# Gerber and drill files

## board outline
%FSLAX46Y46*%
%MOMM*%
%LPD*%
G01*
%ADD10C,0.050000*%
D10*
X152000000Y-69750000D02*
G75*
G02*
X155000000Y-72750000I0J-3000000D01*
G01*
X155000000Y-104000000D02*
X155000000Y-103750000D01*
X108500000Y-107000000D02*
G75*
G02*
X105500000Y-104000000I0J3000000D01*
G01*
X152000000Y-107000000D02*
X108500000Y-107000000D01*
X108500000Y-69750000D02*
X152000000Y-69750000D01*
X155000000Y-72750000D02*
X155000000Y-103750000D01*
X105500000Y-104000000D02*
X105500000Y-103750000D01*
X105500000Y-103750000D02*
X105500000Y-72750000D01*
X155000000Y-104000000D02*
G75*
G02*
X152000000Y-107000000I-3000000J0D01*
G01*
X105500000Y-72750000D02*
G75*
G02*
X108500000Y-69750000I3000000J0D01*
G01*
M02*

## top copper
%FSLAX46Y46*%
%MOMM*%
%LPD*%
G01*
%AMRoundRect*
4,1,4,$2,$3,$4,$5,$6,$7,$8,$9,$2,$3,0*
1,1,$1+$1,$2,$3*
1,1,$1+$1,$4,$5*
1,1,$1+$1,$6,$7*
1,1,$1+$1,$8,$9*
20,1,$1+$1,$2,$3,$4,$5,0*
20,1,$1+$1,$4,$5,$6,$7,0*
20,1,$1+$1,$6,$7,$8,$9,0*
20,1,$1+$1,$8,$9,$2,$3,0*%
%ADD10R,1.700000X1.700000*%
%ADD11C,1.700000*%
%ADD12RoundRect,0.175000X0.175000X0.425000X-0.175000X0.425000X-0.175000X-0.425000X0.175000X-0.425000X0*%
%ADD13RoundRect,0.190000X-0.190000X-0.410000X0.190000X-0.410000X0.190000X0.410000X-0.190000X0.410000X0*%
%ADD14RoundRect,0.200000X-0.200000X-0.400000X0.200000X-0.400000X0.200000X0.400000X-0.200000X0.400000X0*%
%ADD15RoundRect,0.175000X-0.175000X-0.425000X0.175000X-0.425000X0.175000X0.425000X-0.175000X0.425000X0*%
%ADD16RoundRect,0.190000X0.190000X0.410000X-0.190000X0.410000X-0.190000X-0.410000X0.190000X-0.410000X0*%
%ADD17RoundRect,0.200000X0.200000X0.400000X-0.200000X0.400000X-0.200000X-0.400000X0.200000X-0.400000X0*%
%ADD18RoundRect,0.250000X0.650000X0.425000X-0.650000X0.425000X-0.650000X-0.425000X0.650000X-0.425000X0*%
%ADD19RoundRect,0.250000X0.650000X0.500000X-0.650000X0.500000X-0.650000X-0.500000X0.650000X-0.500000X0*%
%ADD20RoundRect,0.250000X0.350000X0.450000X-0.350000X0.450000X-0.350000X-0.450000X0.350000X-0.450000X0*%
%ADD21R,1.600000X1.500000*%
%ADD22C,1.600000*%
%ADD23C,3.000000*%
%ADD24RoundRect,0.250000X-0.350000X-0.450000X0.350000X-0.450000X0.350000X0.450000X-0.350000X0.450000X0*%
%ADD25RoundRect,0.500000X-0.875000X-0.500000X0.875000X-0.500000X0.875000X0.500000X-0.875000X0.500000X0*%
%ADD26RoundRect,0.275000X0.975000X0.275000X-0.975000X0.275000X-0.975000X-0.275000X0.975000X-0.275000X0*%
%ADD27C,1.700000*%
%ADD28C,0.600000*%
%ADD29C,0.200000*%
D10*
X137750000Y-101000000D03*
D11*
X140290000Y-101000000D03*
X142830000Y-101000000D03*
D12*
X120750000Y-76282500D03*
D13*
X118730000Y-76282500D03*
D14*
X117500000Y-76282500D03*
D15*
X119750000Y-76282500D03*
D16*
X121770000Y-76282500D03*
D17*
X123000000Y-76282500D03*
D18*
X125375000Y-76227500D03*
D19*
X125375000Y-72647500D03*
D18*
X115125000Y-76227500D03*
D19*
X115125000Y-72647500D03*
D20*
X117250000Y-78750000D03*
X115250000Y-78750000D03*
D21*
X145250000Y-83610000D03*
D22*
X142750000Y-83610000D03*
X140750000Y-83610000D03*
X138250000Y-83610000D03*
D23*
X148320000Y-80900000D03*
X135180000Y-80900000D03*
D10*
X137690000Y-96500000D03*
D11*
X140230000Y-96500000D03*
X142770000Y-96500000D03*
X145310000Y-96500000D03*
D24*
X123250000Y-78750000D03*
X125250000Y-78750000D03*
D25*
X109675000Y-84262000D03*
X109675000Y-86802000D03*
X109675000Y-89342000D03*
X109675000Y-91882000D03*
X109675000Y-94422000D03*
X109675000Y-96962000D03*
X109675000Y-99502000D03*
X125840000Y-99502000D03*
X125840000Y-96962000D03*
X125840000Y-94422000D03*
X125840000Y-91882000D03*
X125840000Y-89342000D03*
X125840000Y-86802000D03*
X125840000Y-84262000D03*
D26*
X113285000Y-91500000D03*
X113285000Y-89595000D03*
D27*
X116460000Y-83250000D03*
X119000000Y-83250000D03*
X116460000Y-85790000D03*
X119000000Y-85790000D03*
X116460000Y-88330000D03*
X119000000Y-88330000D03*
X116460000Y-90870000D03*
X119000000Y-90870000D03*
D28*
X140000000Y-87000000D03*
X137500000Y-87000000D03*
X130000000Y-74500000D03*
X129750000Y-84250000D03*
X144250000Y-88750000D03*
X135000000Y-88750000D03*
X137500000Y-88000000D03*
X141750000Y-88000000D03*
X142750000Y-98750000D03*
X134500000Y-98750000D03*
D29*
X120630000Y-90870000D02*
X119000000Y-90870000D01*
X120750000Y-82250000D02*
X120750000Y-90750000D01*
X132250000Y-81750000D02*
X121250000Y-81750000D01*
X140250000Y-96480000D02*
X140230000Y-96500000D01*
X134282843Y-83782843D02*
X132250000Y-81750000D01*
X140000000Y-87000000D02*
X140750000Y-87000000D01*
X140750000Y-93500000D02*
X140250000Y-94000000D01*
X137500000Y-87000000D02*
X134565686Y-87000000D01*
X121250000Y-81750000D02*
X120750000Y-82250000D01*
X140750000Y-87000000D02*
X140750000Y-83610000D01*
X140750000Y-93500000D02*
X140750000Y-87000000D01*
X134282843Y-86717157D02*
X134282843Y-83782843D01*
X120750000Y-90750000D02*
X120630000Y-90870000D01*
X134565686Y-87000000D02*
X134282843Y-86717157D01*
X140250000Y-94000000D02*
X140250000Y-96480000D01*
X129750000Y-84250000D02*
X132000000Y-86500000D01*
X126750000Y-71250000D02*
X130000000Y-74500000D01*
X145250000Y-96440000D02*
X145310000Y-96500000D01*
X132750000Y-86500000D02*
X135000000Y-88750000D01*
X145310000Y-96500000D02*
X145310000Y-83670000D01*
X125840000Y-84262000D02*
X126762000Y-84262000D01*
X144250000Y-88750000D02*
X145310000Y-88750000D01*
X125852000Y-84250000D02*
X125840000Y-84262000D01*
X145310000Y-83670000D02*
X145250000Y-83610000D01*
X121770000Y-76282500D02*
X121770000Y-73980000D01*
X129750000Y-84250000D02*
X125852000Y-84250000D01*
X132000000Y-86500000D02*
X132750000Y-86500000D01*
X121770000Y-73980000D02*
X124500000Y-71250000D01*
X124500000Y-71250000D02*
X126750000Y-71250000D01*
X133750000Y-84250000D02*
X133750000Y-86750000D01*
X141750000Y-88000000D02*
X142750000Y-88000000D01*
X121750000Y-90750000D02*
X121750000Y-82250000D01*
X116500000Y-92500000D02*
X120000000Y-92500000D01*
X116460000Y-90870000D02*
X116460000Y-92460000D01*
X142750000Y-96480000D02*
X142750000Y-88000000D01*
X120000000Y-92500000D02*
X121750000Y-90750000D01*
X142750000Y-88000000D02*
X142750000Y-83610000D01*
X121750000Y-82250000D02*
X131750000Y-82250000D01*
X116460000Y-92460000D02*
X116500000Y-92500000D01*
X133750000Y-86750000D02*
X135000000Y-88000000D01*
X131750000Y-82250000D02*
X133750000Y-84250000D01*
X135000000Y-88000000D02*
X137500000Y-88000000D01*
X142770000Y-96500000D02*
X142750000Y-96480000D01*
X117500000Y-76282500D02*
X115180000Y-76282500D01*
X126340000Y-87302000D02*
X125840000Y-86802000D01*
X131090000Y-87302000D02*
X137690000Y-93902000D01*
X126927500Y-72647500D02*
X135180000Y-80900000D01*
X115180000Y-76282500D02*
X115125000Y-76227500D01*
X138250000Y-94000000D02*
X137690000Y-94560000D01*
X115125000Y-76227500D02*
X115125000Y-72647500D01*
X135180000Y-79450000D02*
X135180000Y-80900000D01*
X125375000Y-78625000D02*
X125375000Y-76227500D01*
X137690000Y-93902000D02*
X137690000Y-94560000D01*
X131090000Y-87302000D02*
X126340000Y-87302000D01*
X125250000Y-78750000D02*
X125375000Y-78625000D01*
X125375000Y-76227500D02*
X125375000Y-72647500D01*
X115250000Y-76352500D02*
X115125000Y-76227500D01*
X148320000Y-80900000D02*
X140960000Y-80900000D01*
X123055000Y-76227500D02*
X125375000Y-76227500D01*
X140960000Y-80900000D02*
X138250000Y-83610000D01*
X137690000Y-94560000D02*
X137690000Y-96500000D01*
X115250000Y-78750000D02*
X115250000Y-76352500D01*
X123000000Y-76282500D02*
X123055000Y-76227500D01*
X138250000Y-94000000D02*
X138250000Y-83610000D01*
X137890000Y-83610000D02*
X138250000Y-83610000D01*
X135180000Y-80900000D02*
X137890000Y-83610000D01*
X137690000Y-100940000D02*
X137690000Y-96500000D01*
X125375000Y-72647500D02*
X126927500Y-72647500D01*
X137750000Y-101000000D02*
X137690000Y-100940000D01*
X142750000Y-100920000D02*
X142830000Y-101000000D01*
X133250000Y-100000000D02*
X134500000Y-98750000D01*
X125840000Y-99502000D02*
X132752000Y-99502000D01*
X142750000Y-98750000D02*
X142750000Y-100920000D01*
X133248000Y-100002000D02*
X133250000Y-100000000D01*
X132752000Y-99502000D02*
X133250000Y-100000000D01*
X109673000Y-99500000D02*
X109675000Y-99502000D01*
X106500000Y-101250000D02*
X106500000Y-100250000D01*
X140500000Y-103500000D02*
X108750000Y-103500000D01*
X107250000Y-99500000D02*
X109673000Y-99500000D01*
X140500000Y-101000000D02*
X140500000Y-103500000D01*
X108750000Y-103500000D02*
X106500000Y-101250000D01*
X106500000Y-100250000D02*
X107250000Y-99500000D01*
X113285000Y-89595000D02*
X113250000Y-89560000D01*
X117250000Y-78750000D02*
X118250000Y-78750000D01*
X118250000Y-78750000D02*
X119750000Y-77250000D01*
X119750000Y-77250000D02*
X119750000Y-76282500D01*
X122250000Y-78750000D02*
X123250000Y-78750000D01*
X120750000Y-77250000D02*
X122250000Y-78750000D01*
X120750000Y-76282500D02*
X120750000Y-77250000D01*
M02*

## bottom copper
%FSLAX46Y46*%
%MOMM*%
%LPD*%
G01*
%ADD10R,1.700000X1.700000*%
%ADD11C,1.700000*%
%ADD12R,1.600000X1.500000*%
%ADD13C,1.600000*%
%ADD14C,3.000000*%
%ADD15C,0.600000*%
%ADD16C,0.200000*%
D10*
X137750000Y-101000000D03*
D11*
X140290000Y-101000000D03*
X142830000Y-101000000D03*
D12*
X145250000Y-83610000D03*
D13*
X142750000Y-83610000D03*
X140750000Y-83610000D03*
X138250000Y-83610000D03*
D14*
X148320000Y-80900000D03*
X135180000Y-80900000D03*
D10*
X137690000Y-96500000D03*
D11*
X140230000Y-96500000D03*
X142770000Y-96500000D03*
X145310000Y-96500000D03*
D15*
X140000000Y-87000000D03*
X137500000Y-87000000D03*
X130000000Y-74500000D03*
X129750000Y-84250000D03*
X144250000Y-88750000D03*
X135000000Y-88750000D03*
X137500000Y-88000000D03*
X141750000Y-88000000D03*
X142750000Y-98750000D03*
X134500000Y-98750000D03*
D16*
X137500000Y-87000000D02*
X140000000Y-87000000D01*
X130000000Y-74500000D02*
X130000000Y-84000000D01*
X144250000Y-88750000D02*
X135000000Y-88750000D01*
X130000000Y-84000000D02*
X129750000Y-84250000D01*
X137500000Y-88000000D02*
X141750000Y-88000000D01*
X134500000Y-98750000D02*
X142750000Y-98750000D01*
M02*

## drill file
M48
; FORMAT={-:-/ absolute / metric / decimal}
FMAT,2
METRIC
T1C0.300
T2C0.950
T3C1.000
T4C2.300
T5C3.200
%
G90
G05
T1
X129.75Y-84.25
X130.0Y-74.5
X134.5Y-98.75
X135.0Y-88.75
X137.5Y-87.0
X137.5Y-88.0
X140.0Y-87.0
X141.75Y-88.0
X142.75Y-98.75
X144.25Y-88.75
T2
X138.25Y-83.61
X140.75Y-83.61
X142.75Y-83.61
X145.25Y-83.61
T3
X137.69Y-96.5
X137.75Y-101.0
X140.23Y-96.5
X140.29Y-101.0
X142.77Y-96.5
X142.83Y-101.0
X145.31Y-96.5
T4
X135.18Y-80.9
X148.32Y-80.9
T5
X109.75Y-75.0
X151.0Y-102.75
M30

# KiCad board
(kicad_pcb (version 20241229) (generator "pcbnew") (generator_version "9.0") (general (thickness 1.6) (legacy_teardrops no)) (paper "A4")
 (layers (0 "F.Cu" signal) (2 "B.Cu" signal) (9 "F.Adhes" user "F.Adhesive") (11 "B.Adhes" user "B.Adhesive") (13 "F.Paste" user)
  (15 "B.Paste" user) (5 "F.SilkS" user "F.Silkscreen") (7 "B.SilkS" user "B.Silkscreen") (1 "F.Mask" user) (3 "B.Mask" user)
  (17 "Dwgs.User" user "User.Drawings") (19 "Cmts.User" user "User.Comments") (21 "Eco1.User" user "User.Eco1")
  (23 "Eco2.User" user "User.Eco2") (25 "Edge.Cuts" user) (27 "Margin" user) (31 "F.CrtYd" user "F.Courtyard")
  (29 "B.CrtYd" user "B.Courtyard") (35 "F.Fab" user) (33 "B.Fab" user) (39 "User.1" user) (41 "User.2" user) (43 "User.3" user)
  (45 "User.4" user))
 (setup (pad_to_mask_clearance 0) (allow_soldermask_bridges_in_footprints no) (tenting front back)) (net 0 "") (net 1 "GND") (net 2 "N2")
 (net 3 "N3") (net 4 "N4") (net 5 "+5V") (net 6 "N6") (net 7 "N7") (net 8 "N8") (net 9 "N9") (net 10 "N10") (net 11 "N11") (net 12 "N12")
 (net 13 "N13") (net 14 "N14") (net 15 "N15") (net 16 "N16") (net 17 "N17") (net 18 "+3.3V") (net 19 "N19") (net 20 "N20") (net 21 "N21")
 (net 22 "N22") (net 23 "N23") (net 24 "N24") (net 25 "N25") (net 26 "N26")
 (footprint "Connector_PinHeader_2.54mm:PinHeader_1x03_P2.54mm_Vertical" (layer "F.Cu") (at 137.75 101 90)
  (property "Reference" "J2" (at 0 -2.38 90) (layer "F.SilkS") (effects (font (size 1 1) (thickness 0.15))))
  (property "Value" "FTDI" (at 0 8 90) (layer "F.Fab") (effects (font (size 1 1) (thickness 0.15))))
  (pad "1" thru_hole rect (at 0 0 90) (size 1.7 1.7) (drill 1) (layers "*.Cu" "*.Mask") (remove_unused_layers no) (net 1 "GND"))
  (pad "2" thru_hole circle (at 0 2.54 90) (size 1.7 1.7) (drill 1) (layers "*.Cu" "*.Mask") (remove_unused_layers no) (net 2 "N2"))
  (pad "3" thru_hole circle (at 0 5.08 90) (size 1.7 1.7) (drill 1) (layers "*.Cu" "*.Mask") (remove_unused_layers no) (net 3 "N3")))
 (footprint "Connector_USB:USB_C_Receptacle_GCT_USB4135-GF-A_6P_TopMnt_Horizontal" (layer "F.Cu") (at 120.25 73.25 180)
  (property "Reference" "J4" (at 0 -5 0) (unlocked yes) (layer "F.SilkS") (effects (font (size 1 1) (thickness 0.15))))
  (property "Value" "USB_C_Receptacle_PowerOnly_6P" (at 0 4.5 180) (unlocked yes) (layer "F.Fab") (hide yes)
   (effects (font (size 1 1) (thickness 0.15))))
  (pad "A5" smd roundrect (at -0.5 -3.0325 180) (size 0.7 1.2) (layers "F.Cu" "F.Mask" "F.Paste") (roundrect_rratio 0.25) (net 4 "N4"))
  (pad "A9" smd roundrect (at 1.52 -3.0325) (size 0.76 1.2) (layers "F.Cu" "F.Mask" "F.Paste") (roundrect_rratio 0.25) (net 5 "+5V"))
  (pad "A12" smd roundrect (at 2.75 -3.0325) (size 0.8 1.2) (layers "F.Cu" "F.Mask" "F.Paste") (roundrect_rratio 0.25) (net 1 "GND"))
  (pad "B5" smd roundrect (at 0.5 -3.0325) (size 0.7 1.2) (layers "F.Cu" "F.Mask" "F.Paste") (roundrect_rratio 0.25) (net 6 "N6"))
  (pad "B9" smd roundrect (at -1.52 -3.0325 180) (size 0.76 1.2) (layers "F.Cu" "F.Mask" "F.Paste") (roundrect_rratio 0.25) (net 5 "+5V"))
  (pad "B12" smd roundrect (at -2.75 -3.0325 180) (size 0.8 1.2) (layers "F.Cu" "F.Mask" "F.Paste") (roundrect_rratio 0.25) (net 1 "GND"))
  (pad "S1" smd roundrect (at -5.125 -2.9775 180) (size 1.8 1.35) (layers "F.Cu" "F.Mask" "F.Paste") (roundrect_rratio 0.1851851852)
   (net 1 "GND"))
  (pad "S1" smd roundrect (at -5.125 0.6025 180) (size 1.8 1.5) (layers "F.Cu" "F.Mask" "F.Paste") (roundrect_rratio 0.1666666667)
   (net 1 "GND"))
  (pad "S1" smd roundrect (at 5.125 -2.9775 180) (size 1.8 1.35) (layers "F.Cu" "F.Mask" "F.Paste") (roundrect_rratio 0.1851851852)
   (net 1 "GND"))
  (pad "S1" smd roundrect (at 5.125 0.6025 180) (size 1.8 1.5) (layers "F.Cu" "F.Mask" "F.Paste") (roundrect_rratio 0.1666666667)
   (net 1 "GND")))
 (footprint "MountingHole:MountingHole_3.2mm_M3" (layer "F.Cu") (at 151 102.75)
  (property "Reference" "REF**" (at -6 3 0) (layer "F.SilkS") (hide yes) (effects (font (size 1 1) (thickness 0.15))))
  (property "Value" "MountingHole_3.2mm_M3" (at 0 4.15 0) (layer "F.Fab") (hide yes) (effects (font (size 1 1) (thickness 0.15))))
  (pad "" np_thru_hole circle (at 0 0) (size 3.2 3.2) (drill 3.2) (layers "*.Cu" "*.Mask")))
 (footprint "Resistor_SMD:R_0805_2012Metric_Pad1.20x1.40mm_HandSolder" (layer "F.Cu") (at 116.25 78.75 180)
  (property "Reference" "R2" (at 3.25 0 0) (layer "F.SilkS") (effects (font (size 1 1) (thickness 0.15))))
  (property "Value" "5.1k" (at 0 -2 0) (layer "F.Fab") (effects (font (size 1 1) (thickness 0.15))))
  (pad "1" smd roundrect (at -1 0 180) (size 1.2 1.4) (layers "F.Cu" "F.Mask" "F.Paste") (roundrect_rratio 0.208333) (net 6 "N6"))
  (pad "2" smd roundrect (at 1 0 180) (size 1.2 1.4) (layers "F.Cu" "F.Mask" "F.Paste") (roundrect_rratio 0.208333) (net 1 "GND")))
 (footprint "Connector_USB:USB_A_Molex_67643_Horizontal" (layer "F.Cu") (at 145.25 83.61 180)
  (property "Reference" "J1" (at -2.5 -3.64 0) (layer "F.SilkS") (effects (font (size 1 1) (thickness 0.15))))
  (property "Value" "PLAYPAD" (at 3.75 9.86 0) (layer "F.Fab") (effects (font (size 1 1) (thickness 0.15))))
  (pad "1" thru_hole rect (at 0 0 180) (size 1.6 1.5) (drill 0.95) (layers "*.Cu" "*.Mask") (remove_unused_layers no) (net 5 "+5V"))
  (pad "2" thru_hole circle (at 2.5 0 180) (size 1.6 1.6) (drill 0.95) (layers "*.Cu" "*.Mask") (remove_unused_layers no) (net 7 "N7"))
  (pad "3" thru_hole circle (at 4.5 0 180) (size 1.6 1.6) (drill 0.95) (layers "*.Cu" "*.Mask") (remove_unused_layers no) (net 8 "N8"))
  (pad "4" thru_hole circle (at 7 0 180) (size 1.6 1.6) (drill 0.95) (layers "*.Cu" "*.Mask") (remove_unused_layers no) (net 1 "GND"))
  (pad "5" thru_hole circle (at -3.07 2.71 180) (size 3 3) (drill 2.3) (layers "*.Cu" "*.Mask") (remove_unused_layers no) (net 1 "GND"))
  (pad "5" thru_hole circle (at 10.07 2.71 180) (size 3 3) (drill 2.3) (layers "*.Cu" "*.Mask") (remove_unused_layers no) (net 1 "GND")))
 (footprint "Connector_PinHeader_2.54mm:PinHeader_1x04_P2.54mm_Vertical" (layer "F.Cu") (at 137.69 96.5 90)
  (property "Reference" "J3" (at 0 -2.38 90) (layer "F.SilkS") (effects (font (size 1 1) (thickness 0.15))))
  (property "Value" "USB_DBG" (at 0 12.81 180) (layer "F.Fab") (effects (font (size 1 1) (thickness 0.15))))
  (pad "1" thru_hole rect (at 0 0 90) (size 1.7 1.7) (drill 1) (layers "*.Cu" "*.Mask") (remove_unused_layers no) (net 1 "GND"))
  (pad "2" thru_hole circle (at 0 2.54 90) (size 1.7 1.7) (drill 1) (layers "*.Cu" "*.Mask") (remove_unused_layers no) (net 8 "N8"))
  (pad "3" thru_hole circle (at 0 5.08 90) (size 1.7 1.7) (drill 1) (layers "*.Cu" "*.Mask") (remove_unused_layers no) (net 7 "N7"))
  (pad "4" thru_hole circle (at 0 7.62 90) (size 1.7 1.7) (drill 1) (layers "*.Cu" "*.Mask") (remove_unused_layers no) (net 5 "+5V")))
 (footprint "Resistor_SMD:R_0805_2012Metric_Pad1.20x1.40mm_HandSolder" (layer "F.Cu") (at 124.25 78.75)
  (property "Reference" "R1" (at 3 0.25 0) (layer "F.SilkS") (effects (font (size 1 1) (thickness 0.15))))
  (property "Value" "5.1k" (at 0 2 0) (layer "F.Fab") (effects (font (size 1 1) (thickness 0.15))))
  (pad "1" smd roundrect (at -1 0) (size 1.2 1.4) (layers "F.Cu" "F.Mask" "F.Paste") (roundrect_rratio 0.208333) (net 4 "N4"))
  (pad "2" smd roundrect (at 1 0) (size 1.2 1.4) (layers "F.Cu" "F.Mask" "F.Paste") (roundrect_rratio 0.208333) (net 1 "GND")))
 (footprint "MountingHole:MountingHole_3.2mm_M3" (layer "F.Cu") (at 109.75 75)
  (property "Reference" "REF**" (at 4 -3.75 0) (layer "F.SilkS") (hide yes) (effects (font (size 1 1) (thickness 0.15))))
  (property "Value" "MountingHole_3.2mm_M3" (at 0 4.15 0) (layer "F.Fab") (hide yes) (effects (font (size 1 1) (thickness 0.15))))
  (pad "" np_thru_hole circle (at 0 0) (size 3.2 3.2) (drill 3.2) (layers "*.Cu" "*.Mask")))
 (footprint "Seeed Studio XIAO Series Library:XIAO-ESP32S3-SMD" (layer "F.Cu") (at 117.736364 91.835)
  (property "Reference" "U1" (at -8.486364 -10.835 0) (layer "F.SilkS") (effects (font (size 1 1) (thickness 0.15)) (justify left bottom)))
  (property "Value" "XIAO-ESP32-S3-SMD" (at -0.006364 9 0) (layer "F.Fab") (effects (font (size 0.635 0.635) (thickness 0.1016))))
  (pad "1" smd roundrect (at -8.061364 -7.573) (size 2.75 2) (layers "F.Cu" "F.Mask" "F.Paste") (roundrect_rratio 0.25) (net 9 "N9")
   (solder_mask_margin 0.0508) (thermal_bridge_angle 45))
  (pad "2" smd roundrect (at -8.061364 -5.033) (size 2.75 2) (layers "F.Cu" "F.Mask" "F.Paste") (roundrect_rratio 0.25) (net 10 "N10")
   (solder_mask_margin 0.0508) (thermal_bridge_angle 45))
  (pad "3" smd roundrect (at -8.061364 -2.493) (size 2.75 2) (layers "F.Cu" "F.Mask" "F.Paste") (roundrect_rratio 0.25) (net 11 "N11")
   (solder_mask_margin 0.0508) (thermal_bridge_angle 45))
  (pad "4" smd roundrect (at -8.061364 0.047) (size 2.75 2) (layers "F.Cu" "F.Mask" "F.Paste") (roundrect_rratio 0.25) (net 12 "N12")
   (solder_mask_margin 0.0508) (thermal_bridge_angle 45))
  (pad "5" smd roundrect (at -8.061364 2.587) (size 2.75 2) (layers "F.Cu" "F.Mask" "F.Paste") (roundrect_rratio 0.25) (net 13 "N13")
   (solder_mask_margin 0.0508) (thermal_bridge_angle 45))
  (pad "6" smd roundrect (at -8.061364 5.127) (size 2.75 2) (layers "F.Cu" "F.Mask" "F.Paste") (roundrect_rratio 0.25) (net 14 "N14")
   (solder_mask_margin 0.0508) (thermal_bridge_angle 45))
  (pad "7" smd roundrect (at -8.061364 7.667) (size 2.75 2) (layers "F.Cu" "F.Mask" "F.Paste") (roundrect_rratio 0.25) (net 2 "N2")
   (solder_mask_margin 0.0508) (thermal_bridge_angle 45))
  (pad "8" smd roundrect (at 8.103636 7.667) (size 2.75 2) (layers "F.Cu" "F.Mask" "F.Paste") (roundrect_rratio 0.25) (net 3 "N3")
   (solder_mask_margin 0.0508) (thermal_bridge_angle 45))
  (pad "9" smd roundrect (at 8.103636 5.127) (size 2.75 2) (layers "F.Cu" "F.Mask" "F.Paste") (roundrect_rratio 0.25) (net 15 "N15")
   (solder_mask_margin 0.0508) (thermal_bridge_angle 45))
  (pad "10" smd roundrect (at 8.103636 2.587) (size 2.75 2) (layers "F.Cu" "F.Mask" "F.Paste") (roundrect_rratio 0.25) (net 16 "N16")
   (solder_mask_margin 0.0508) (thermal_bridge_angle 45))
  (pad "11" smd roundrect (at 8.103636 0.047) (size 2.75 2) (layers "F.Cu" "F.Mask" "F.Paste") (roundrect_rratio 0.25) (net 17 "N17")
   (solder_mask_margin 0.0508) (thermal_bridge_angle 45))
  (pad "12" smd roundrect (at 8.103636 -2.493) (size 2.75 2) (layers "F.Cu" "F.Mask" "F.Paste") (roundrect_rratio 0.25) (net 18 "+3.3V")
   (solder_mask_margin 0.0508) (thermal_bridge_angle 45))
  (pad "13" smd roundrect (at 8.103636 -5.033) (size 2.75 2) (layers "F.Cu" "F.Mask" "F.Paste") (roundrect_rratio 0.25) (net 1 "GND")
   (solder_mask_margin 0.0508) (thermal_bridge_angle 45))
  (pad "14" smd roundrect (at 8.103636 -7.573) (size 2.75 2) (layers "F.Cu" "F.Mask" "F.Paste") (roundrect_rratio 0.25) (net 5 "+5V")
   (solder_mask_margin 0.0508) (thermal_bridge_angle 45))
  (pad "15" smd roundrect (at -4.451364 -0.335 180) (size 2.5 1.1) (layers "F.Cu" "F.Mask" "F.Paste") (roundrect_rratio 0.25) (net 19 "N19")
   (solder_mask_margin 0.0508) (thermal_bridge_angle 45))
  (pad "16" smd roundrect (at -4.451364 -2.24 180) (size 2.5 1.1) (layers "F.Cu" "F.Mask" "F.Paste") (roundrect_rratio 0.25) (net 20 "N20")
   (solder_mask_margin 0.0508) (thermal_bridge_angle 45))
  (pad "17" smd circle (at -1.276364 -8.585) (size 1.7 1.7) (layers "F.Cu" "F.Mask" "F.Paste") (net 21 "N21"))
  (pad "18" smd circle (at 1.263636 -8.585) (size 1.7 1.7) (layers "F.Cu" "F.Mask" "F.Paste") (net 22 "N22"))
  (pad "19" smd circle (at -1.276364 -6.045) (size 1.7 1.7) (layers "F.Cu" "F.Mask" "F.Paste") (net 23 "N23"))
  (pad "20" smd circle (at 1.263636 -6.045) (size 1.7 1.7) (layers "F.Cu" "F.Mask" "F.Paste") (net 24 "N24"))
  (pad "21" smd circle (at -1.276364 -3.505) (size 1.7 1.7) (layers "F.Cu" "F.Mask" "F.Paste") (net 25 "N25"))
  (pad "22" smd circle (at 1.263636 -3.505) (size 1.7 1.7) (layers "F.Cu" "F.Mask" "F.Paste") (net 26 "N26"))
  (pad "23" smd circle (at -1.276364 -0.965) (size 1.7 1.7) (layers "F.Cu" "F.Mask" "F.Paste") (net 7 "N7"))
  (pad "24" smd circle (at 1.263636 -0.965) (size 1.7 1.7) (layers "F.Cu" "F.Mask" "F.Paste") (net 8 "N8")))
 (gr_arc (start 152 69.75) (mid 154.12132 70.62868) (end 155 72.75) (stroke (width 0.05) (type default)) (layer "Edge.Cuts"))
 (gr_line (start 155 104) (end 155 103.75) (stroke (width 0.05) (type default)) (layer "Edge.Cuts"))
 (gr_arc (start 108.5 107) (mid 106.37868 106.12132) (end 105.5 104) (stroke (width 0.05) (type default)) (layer "Edge.Cuts"))
 (gr_line (start 152 107) (end 108.5 107) (stroke (width 0.05) (type default)) (layer "Edge.Cuts"))
 (gr_line (start 108.5 69.75) (end 152 69.75) (stroke (width 0.05) (type default)) (layer "Edge.Cuts"))
 (gr_line (start 155 72.75) (end 155 103.75) (stroke (width 0.05) (type default)) (layer "Edge.Cuts"))
 (gr_line (start 105.5 104) (end 105.5 103.75) (stroke (width 0.05) (type default)) (layer "Edge.Cuts"))
 (gr_line (start 105.5 103.75) (end 105.5 72.75) (stroke (width 0.05) (type default)) (layer "Edge.Cuts"))
 (gr_arc (start 155 104) (mid 154.12132 106.12132) (end 152 107) (stroke (width 0.05) (type default)) (layer "Edge.Cuts"))
 (gr_arc (start 105.5 72.75) (mid 106.37868 70.62868) (end 108.5 69.75) (stroke (width 0.05) (type default)) (layer "Edge.Cuts"))
 (segment (start 120.63 90.87) (end 119 90.87) (width 0.2) (layer "F.Cu") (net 8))
 (segment (start 120.75 82.25) (end 120.75 90.75) (width 0.2) (layer "F.Cu") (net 8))
 (segment (start 132.25 81.75) (end 121.25 81.75) (width 0.2) (layer "F.Cu") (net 8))
 (segment (start 140.25 96.48) (end 140.23 96.5) (width 0.2) (layer "F.Cu") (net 8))
 (segment (start 134.282843 83.782843) (end 132.25 81.75) (width 0.2) (layer "F.Cu") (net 8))
 (segment (start 140 87) (end 140.75 87) (width 0.2) (layer "F.Cu") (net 8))
 (segment (start 140.75 93.5) (end 140.25 94) (width 0.2) (layer "F.Cu") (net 8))
 (segment (start 137.5 87) (end 134.565686 87) (width 0.2) (layer "F.Cu") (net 8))
 (segment (start 121.25 81.75) (end 120.75 82.25) (width 0.2) (layer "F.Cu") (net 8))
 (segment (start 140.75 87) (end 140.75 83.61) (width 0.2) (layer "F.Cu") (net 8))
 (segment (start 140.75 93.5) (end 140.75 87) (width 0.2) (layer "F.Cu") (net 8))
 (segment (start 134.282843 86.717157) (end 134.282843 83.782843) (width 0.2) (layer "F.Cu") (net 8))
 (segment (start 120.75 90.75) (end 120.63 90.87) (width 0.2) (layer "F.Cu") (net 8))
 (segment (start 134.565686 87) (end 134.282843 86.717157) (width 0.2) (layer "F.Cu") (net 8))
 (segment (start 140.25 94) (end 140.25 96.48) (width 0.2) (layer "F.Cu") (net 8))
 (via (at 140 87) (size 0.6) (drill 0.3) (layers "F.Cu" "B.Cu") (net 8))
 (via (at 137.5 87) (size 0.6) (drill 0.3) (layers "F.Cu" "B.Cu") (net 8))
 (segment (start 137.5 87) (end 140 87) (width 0.2) (layer "B.Cu") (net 8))
 (segment (start 129.75 84.25) (end 132 86.5) (width 0.2) (layer "F.Cu") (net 5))
 (segment (start 126.75 71.25) (end 130 74.5) (width 0.2) (layer "F.Cu") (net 5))
 (segment (start 145.25 96.44) (end 145.31 96.5) (width 0.2) (layer "F.Cu") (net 5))
 (segment (start 132.75 86.5) (end 135 88.75) (width 0.2) (layer "F.Cu") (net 5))
 (segment (start 145.31 96.5) (end 145.31 83.67) (width 0.2) (layer "F.Cu") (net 5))
 (segment (start 125.84 84.262) (end 126.762 84.262) (width 0.2) (layer "F.Cu") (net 5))
 (segment (start 144.25 88.75) (end 145.31 88.75) (width 0.2) (layer "F.Cu") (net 5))
 (segment (start 125.852 84.25) (end 125.84 84.262) (width 0.2) (layer "F.Cu") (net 5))
 (segment (start 145.31 83.67) (end 145.25 83.61) (width 0.2) (layer "F.Cu") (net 5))
 (segment (start 121.77 76.2825) (end 121.77 73.98) (width 0.2) (layer "F.Cu") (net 5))
 (segment (start 129.75 84.25) (end 125.852 84.25) (width 0.2) (layer "F.Cu") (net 5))
 (segment (start 132 86.5) (end 132.75 86.5) (width 0.2) (layer "F.Cu") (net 5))
 (segment (start 121.77 73.98) (end 124.5 71.25) (width 0.2) (layer "F.Cu") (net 5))
 (segment (start 124.5 71.25) (end 126.75 71.25) (width 0.2) (layer "F.Cu") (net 5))
 (via (at 130 74.5) (size 0.6) (drill 0.3) (layers "F.Cu" "B.Cu") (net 5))
 (via (at 129.75 84.25) (size 0.6) (drill 0.3) (layers "F.Cu" "B.Cu") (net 5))
 (via (at 144.25 88.75) (size 0.6) (drill 0.3) (layers "F.Cu" "B.Cu") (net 5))
 (via (at 135 88.75) (size 0.6) (drill 0.3) (layers "F.Cu" "B.Cu") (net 5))
 (segment (start 130 74.5) (end 130 84) (width 0.2) (layer "B.Cu") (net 5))
 (segment (start 144.25 88.75) (end 135 88.75) (width 0.2) (layer "B.Cu") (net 5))
 (segment (start 130 84) (end 129.75 84.25) (width 0.2) (layer "B.Cu") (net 5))
 (segment (start 133.75 84.25) (end 133.75 86.75) (width 0.2) (layer "F.Cu") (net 7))
 (segment (start 141.75 88) (end 142.75 88) (width 0.2) (layer "F.Cu") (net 7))
 (segment (start 121.75 90.75) (end 121.75 82.25) (width 0.2) (layer "F.Cu") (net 7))
 (segment (start 116.5 92.5) (end 120 92.5) (width 0.2) (layer "F.Cu") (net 7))
 (segment (start 116.46 90.87) (end 116.46 92.46) (width 0.2) (layer "F.Cu") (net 7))
 (segment (start 142.75 96.48) (end 142.75 88) (width 0.2) (layer "F.Cu") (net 7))
 (segment (start 120 92.5) (end 121.75 90.75) (width 0.2) (layer "F.Cu") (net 7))
 (segment (start 142.75 88) (end 142.75 83.61) (width 0.2) (layer "F.Cu") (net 7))
 (segment (start 121.75 82.25) (end 131.75 82.25) (width 0.2) (layer "F.Cu") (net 7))
 (segment (start 116.46 92.46) (end 116.5 92.5) (width 0.2) (layer "F.Cu") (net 7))
 (segment (start 133.75 86.75) (end 135 88) (width 0.2) (layer "F.Cu") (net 7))
 (segment (start 131.75 82.25) (end 133.75 84.25) (width 0.2) (layer "F.Cu") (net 7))
 (segment (start 135 88) (end 137.5 88) (width 0.2) (layer "F.Cu") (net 7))
 (segment (start 142.77 96.5) (end 142.75 96.48) (width 0.2) (layer "F.Cu") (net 7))
 (via (at 137.5 88) (size 0.6) (drill 0.3) (layers "F.Cu" "B.Cu") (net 7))
 (via (at 141.75 88) (size 0.6) (drill 0.3) (layers "F.Cu" "B.Cu") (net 7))
 (segment (start 137.5 88) (end 141.75 88) (width 0.2) (layer "B.Cu") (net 7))
 (segment (start 117.5 76.2825) (end 115.18 76.2825) (width 0.2) (layer "F.Cu") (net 1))
 (segment (start 126.34 87.302) (end 125.84 86.802) (width 0.2) (layer "F.Cu") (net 1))
 (segment (start 131.09 87.302) (end 137.69 93.902) (width 0.2) (layer "F.Cu") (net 1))
 (segment (start 126.9275 72.6475) (end 135.18 80.9) (width 0.2) (layer "F.Cu") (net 1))
 (segment (start 115.18 76.2825) (end 115.125 76.2275) (width 0.2) (layer "F.Cu") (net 1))
 (segment (start 138.25 94) (end 137.69 94.56) (width 0.2) (layer "F.Cu") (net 1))
 (segment (start 115.125 76.2275) (end 115.125 72.6475) (width 0.2) (layer "F.Cu") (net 1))
 (segment (start 135.18 79.45) (end 135.18 80.9) (width 0.2) (layer "F.Cu") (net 1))
 (segment (start 125.375 78.625) (end 125.375 76.2275) (width 0.2) (layer "F.Cu") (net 1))
 (segment (start 137.69 93.902) (end 137.69 94.56) (width 0.2) (layer "F.Cu") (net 1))
 (segment (start 131.09 87.302) (end 126.34 87.302) (width 0.2) (layer "F.Cu") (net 1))
 (segment (start 125.25 78.75) (end 125.375 78.625) (width 0.2) (layer "F.Cu") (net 1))
 (segment (start 125.375 76.2275) (end 125.375 72.6475) (width 0.2) (layer "F.Cu") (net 1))
 (segment (start 115.25 76.3525) (end 115.125 76.2275) (width 0.2) (layer "F.Cu") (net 1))
 (segment (start 148.32 80.9) (end 140.96 80.9) (width 0.2) (layer "F.Cu") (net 1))
 (segment (start 123.055 76.2275) (end 125.375 76.2275) (width 0.2) (layer "F.Cu") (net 1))
 (segment (start 140.96 80.9) (end 138.25 83.61) (width 0.2) (layer "F.Cu") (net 1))
 (segment (start 137.69 94.56) (end 137.69 96.5) (width 0.2) (layer "F.Cu") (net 1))
 (segment (start 115.25 78.75) (end 115.25 76.3525) (width 0.2) (layer "F.Cu") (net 1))
 (segment (start 123 76.2825) (end 123.055 76.2275) (width 0.2) (layer "F.Cu") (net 1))
 (segment (start 138.25 94) (end 138.25 83.61) (width 0.2) (layer "F.Cu") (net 1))
 (segment (start 137.89 83.61) (end 138.25 83.61) (width 0.2) (layer "F.Cu") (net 1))
 (segment (start 135.18 80.9) (end 137.89 83.61) (width 0.2) (layer "F.Cu") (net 1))
 (segment (start 137.69 100.94) (end 137.69 96.5) (width 0.2) (layer "F.Cu") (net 1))
 (segment (start 125.375 72.6475) (end 126.9275 72.6475) (width 0.2) (layer "F.Cu") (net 1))
 (segment (start 137.75 101) (end 137.69 100.94) (width 0.2) (layer "F.Cu") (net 1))
 (segment (start 142.75 100.92) (end 142.83 101) (width 0.2) (layer "F.Cu") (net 3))
 (segment (start 133.25 100) (end 134.5 98.75) (width 0.2) (layer "F.Cu") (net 3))
 (segment (start 125.84 99.502) (end 132.752 99.502) (width 0.2) (layer "F.Cu") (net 3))
 (segment (start 142.75 98.75) (end 142.75 100.92) (width 0.2) (layer "F.Cu") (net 3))
 (segment (start 133.248 100.002) (end 133.25 100) (width 0.2) (layer "F.Cu") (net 3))
 (segment (start 132.752 99.502) (end 133.25 100) (width 0.2) (layer "F.Cu") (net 3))
 (via (at 142.75 98.75) (size 0.6) (drill 0.3) (layers "F.Cu" "B.Cu") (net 3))
 (via (at 134.5 98.75) (size 0.6) (drill 0.3) (layers "F.Cu" "B.Cu") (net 3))
 (segment (start 134.5 98.75) (end 142.75 98.75) (width 0.2) (layer "B.Cu") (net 3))
 (segment (start 109.673 99.5) (end 109.675 99.502) (width 0.2) (layer "F.Cu") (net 2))
 (segment (start 106.5 101.25) (end 106.5 100.25) (width 0.2) (layer "F.Cu") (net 2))
 (segment (start 140.5 103.5) (end 108.75 103.5) (width 0.2) (layer "F.Cu") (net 2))
 (segment (start 107.25 99.5) (end 109.673 99.5) (width 0.2) (layer "F.Cu") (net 2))
 (segment (start 140.5 101) (end 140.5 103.5) (width 0.2) (layer "F.Cu") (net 2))
 (segment (start 108.75 103.5) (end 106.5 101.25) (width 0.2) (layer "F.Cu") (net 2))
 (segment (start 106.5 100.25) (end 107.25 99.5) (width 0.2) (layer "F.Cu") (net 2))
 (segment (start 113.285 89.595) (end 113.25 89.56) (width 0.2) (layer "F.Cu") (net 20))
 (segment (start 117.25 78.75) (end 118.25 78.75) (width 0.2) (layer "F.Cu") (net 6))
 (segment (start 118.25 78.75) (end 119.75 77.25) (width 0.2) (layer "F.Cu") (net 6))
 (segment (start 119.75 77.25) (end 119.75 76.2825) (width 0.2) (layer "F.Cu") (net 6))
 (segment (start 122.25 78.75) (end 123.25 78.75) (width 0.2) (layer "F.Cu") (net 4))
 (segment (start 120.75 77.25) (end 122.25 78.75) (width 0.2) (layer "F.Cu") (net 4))
 (segment (start 120.75 76.2825) (end 120.75 77.25) (width 0.2) (layer "F.Cu") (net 4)))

